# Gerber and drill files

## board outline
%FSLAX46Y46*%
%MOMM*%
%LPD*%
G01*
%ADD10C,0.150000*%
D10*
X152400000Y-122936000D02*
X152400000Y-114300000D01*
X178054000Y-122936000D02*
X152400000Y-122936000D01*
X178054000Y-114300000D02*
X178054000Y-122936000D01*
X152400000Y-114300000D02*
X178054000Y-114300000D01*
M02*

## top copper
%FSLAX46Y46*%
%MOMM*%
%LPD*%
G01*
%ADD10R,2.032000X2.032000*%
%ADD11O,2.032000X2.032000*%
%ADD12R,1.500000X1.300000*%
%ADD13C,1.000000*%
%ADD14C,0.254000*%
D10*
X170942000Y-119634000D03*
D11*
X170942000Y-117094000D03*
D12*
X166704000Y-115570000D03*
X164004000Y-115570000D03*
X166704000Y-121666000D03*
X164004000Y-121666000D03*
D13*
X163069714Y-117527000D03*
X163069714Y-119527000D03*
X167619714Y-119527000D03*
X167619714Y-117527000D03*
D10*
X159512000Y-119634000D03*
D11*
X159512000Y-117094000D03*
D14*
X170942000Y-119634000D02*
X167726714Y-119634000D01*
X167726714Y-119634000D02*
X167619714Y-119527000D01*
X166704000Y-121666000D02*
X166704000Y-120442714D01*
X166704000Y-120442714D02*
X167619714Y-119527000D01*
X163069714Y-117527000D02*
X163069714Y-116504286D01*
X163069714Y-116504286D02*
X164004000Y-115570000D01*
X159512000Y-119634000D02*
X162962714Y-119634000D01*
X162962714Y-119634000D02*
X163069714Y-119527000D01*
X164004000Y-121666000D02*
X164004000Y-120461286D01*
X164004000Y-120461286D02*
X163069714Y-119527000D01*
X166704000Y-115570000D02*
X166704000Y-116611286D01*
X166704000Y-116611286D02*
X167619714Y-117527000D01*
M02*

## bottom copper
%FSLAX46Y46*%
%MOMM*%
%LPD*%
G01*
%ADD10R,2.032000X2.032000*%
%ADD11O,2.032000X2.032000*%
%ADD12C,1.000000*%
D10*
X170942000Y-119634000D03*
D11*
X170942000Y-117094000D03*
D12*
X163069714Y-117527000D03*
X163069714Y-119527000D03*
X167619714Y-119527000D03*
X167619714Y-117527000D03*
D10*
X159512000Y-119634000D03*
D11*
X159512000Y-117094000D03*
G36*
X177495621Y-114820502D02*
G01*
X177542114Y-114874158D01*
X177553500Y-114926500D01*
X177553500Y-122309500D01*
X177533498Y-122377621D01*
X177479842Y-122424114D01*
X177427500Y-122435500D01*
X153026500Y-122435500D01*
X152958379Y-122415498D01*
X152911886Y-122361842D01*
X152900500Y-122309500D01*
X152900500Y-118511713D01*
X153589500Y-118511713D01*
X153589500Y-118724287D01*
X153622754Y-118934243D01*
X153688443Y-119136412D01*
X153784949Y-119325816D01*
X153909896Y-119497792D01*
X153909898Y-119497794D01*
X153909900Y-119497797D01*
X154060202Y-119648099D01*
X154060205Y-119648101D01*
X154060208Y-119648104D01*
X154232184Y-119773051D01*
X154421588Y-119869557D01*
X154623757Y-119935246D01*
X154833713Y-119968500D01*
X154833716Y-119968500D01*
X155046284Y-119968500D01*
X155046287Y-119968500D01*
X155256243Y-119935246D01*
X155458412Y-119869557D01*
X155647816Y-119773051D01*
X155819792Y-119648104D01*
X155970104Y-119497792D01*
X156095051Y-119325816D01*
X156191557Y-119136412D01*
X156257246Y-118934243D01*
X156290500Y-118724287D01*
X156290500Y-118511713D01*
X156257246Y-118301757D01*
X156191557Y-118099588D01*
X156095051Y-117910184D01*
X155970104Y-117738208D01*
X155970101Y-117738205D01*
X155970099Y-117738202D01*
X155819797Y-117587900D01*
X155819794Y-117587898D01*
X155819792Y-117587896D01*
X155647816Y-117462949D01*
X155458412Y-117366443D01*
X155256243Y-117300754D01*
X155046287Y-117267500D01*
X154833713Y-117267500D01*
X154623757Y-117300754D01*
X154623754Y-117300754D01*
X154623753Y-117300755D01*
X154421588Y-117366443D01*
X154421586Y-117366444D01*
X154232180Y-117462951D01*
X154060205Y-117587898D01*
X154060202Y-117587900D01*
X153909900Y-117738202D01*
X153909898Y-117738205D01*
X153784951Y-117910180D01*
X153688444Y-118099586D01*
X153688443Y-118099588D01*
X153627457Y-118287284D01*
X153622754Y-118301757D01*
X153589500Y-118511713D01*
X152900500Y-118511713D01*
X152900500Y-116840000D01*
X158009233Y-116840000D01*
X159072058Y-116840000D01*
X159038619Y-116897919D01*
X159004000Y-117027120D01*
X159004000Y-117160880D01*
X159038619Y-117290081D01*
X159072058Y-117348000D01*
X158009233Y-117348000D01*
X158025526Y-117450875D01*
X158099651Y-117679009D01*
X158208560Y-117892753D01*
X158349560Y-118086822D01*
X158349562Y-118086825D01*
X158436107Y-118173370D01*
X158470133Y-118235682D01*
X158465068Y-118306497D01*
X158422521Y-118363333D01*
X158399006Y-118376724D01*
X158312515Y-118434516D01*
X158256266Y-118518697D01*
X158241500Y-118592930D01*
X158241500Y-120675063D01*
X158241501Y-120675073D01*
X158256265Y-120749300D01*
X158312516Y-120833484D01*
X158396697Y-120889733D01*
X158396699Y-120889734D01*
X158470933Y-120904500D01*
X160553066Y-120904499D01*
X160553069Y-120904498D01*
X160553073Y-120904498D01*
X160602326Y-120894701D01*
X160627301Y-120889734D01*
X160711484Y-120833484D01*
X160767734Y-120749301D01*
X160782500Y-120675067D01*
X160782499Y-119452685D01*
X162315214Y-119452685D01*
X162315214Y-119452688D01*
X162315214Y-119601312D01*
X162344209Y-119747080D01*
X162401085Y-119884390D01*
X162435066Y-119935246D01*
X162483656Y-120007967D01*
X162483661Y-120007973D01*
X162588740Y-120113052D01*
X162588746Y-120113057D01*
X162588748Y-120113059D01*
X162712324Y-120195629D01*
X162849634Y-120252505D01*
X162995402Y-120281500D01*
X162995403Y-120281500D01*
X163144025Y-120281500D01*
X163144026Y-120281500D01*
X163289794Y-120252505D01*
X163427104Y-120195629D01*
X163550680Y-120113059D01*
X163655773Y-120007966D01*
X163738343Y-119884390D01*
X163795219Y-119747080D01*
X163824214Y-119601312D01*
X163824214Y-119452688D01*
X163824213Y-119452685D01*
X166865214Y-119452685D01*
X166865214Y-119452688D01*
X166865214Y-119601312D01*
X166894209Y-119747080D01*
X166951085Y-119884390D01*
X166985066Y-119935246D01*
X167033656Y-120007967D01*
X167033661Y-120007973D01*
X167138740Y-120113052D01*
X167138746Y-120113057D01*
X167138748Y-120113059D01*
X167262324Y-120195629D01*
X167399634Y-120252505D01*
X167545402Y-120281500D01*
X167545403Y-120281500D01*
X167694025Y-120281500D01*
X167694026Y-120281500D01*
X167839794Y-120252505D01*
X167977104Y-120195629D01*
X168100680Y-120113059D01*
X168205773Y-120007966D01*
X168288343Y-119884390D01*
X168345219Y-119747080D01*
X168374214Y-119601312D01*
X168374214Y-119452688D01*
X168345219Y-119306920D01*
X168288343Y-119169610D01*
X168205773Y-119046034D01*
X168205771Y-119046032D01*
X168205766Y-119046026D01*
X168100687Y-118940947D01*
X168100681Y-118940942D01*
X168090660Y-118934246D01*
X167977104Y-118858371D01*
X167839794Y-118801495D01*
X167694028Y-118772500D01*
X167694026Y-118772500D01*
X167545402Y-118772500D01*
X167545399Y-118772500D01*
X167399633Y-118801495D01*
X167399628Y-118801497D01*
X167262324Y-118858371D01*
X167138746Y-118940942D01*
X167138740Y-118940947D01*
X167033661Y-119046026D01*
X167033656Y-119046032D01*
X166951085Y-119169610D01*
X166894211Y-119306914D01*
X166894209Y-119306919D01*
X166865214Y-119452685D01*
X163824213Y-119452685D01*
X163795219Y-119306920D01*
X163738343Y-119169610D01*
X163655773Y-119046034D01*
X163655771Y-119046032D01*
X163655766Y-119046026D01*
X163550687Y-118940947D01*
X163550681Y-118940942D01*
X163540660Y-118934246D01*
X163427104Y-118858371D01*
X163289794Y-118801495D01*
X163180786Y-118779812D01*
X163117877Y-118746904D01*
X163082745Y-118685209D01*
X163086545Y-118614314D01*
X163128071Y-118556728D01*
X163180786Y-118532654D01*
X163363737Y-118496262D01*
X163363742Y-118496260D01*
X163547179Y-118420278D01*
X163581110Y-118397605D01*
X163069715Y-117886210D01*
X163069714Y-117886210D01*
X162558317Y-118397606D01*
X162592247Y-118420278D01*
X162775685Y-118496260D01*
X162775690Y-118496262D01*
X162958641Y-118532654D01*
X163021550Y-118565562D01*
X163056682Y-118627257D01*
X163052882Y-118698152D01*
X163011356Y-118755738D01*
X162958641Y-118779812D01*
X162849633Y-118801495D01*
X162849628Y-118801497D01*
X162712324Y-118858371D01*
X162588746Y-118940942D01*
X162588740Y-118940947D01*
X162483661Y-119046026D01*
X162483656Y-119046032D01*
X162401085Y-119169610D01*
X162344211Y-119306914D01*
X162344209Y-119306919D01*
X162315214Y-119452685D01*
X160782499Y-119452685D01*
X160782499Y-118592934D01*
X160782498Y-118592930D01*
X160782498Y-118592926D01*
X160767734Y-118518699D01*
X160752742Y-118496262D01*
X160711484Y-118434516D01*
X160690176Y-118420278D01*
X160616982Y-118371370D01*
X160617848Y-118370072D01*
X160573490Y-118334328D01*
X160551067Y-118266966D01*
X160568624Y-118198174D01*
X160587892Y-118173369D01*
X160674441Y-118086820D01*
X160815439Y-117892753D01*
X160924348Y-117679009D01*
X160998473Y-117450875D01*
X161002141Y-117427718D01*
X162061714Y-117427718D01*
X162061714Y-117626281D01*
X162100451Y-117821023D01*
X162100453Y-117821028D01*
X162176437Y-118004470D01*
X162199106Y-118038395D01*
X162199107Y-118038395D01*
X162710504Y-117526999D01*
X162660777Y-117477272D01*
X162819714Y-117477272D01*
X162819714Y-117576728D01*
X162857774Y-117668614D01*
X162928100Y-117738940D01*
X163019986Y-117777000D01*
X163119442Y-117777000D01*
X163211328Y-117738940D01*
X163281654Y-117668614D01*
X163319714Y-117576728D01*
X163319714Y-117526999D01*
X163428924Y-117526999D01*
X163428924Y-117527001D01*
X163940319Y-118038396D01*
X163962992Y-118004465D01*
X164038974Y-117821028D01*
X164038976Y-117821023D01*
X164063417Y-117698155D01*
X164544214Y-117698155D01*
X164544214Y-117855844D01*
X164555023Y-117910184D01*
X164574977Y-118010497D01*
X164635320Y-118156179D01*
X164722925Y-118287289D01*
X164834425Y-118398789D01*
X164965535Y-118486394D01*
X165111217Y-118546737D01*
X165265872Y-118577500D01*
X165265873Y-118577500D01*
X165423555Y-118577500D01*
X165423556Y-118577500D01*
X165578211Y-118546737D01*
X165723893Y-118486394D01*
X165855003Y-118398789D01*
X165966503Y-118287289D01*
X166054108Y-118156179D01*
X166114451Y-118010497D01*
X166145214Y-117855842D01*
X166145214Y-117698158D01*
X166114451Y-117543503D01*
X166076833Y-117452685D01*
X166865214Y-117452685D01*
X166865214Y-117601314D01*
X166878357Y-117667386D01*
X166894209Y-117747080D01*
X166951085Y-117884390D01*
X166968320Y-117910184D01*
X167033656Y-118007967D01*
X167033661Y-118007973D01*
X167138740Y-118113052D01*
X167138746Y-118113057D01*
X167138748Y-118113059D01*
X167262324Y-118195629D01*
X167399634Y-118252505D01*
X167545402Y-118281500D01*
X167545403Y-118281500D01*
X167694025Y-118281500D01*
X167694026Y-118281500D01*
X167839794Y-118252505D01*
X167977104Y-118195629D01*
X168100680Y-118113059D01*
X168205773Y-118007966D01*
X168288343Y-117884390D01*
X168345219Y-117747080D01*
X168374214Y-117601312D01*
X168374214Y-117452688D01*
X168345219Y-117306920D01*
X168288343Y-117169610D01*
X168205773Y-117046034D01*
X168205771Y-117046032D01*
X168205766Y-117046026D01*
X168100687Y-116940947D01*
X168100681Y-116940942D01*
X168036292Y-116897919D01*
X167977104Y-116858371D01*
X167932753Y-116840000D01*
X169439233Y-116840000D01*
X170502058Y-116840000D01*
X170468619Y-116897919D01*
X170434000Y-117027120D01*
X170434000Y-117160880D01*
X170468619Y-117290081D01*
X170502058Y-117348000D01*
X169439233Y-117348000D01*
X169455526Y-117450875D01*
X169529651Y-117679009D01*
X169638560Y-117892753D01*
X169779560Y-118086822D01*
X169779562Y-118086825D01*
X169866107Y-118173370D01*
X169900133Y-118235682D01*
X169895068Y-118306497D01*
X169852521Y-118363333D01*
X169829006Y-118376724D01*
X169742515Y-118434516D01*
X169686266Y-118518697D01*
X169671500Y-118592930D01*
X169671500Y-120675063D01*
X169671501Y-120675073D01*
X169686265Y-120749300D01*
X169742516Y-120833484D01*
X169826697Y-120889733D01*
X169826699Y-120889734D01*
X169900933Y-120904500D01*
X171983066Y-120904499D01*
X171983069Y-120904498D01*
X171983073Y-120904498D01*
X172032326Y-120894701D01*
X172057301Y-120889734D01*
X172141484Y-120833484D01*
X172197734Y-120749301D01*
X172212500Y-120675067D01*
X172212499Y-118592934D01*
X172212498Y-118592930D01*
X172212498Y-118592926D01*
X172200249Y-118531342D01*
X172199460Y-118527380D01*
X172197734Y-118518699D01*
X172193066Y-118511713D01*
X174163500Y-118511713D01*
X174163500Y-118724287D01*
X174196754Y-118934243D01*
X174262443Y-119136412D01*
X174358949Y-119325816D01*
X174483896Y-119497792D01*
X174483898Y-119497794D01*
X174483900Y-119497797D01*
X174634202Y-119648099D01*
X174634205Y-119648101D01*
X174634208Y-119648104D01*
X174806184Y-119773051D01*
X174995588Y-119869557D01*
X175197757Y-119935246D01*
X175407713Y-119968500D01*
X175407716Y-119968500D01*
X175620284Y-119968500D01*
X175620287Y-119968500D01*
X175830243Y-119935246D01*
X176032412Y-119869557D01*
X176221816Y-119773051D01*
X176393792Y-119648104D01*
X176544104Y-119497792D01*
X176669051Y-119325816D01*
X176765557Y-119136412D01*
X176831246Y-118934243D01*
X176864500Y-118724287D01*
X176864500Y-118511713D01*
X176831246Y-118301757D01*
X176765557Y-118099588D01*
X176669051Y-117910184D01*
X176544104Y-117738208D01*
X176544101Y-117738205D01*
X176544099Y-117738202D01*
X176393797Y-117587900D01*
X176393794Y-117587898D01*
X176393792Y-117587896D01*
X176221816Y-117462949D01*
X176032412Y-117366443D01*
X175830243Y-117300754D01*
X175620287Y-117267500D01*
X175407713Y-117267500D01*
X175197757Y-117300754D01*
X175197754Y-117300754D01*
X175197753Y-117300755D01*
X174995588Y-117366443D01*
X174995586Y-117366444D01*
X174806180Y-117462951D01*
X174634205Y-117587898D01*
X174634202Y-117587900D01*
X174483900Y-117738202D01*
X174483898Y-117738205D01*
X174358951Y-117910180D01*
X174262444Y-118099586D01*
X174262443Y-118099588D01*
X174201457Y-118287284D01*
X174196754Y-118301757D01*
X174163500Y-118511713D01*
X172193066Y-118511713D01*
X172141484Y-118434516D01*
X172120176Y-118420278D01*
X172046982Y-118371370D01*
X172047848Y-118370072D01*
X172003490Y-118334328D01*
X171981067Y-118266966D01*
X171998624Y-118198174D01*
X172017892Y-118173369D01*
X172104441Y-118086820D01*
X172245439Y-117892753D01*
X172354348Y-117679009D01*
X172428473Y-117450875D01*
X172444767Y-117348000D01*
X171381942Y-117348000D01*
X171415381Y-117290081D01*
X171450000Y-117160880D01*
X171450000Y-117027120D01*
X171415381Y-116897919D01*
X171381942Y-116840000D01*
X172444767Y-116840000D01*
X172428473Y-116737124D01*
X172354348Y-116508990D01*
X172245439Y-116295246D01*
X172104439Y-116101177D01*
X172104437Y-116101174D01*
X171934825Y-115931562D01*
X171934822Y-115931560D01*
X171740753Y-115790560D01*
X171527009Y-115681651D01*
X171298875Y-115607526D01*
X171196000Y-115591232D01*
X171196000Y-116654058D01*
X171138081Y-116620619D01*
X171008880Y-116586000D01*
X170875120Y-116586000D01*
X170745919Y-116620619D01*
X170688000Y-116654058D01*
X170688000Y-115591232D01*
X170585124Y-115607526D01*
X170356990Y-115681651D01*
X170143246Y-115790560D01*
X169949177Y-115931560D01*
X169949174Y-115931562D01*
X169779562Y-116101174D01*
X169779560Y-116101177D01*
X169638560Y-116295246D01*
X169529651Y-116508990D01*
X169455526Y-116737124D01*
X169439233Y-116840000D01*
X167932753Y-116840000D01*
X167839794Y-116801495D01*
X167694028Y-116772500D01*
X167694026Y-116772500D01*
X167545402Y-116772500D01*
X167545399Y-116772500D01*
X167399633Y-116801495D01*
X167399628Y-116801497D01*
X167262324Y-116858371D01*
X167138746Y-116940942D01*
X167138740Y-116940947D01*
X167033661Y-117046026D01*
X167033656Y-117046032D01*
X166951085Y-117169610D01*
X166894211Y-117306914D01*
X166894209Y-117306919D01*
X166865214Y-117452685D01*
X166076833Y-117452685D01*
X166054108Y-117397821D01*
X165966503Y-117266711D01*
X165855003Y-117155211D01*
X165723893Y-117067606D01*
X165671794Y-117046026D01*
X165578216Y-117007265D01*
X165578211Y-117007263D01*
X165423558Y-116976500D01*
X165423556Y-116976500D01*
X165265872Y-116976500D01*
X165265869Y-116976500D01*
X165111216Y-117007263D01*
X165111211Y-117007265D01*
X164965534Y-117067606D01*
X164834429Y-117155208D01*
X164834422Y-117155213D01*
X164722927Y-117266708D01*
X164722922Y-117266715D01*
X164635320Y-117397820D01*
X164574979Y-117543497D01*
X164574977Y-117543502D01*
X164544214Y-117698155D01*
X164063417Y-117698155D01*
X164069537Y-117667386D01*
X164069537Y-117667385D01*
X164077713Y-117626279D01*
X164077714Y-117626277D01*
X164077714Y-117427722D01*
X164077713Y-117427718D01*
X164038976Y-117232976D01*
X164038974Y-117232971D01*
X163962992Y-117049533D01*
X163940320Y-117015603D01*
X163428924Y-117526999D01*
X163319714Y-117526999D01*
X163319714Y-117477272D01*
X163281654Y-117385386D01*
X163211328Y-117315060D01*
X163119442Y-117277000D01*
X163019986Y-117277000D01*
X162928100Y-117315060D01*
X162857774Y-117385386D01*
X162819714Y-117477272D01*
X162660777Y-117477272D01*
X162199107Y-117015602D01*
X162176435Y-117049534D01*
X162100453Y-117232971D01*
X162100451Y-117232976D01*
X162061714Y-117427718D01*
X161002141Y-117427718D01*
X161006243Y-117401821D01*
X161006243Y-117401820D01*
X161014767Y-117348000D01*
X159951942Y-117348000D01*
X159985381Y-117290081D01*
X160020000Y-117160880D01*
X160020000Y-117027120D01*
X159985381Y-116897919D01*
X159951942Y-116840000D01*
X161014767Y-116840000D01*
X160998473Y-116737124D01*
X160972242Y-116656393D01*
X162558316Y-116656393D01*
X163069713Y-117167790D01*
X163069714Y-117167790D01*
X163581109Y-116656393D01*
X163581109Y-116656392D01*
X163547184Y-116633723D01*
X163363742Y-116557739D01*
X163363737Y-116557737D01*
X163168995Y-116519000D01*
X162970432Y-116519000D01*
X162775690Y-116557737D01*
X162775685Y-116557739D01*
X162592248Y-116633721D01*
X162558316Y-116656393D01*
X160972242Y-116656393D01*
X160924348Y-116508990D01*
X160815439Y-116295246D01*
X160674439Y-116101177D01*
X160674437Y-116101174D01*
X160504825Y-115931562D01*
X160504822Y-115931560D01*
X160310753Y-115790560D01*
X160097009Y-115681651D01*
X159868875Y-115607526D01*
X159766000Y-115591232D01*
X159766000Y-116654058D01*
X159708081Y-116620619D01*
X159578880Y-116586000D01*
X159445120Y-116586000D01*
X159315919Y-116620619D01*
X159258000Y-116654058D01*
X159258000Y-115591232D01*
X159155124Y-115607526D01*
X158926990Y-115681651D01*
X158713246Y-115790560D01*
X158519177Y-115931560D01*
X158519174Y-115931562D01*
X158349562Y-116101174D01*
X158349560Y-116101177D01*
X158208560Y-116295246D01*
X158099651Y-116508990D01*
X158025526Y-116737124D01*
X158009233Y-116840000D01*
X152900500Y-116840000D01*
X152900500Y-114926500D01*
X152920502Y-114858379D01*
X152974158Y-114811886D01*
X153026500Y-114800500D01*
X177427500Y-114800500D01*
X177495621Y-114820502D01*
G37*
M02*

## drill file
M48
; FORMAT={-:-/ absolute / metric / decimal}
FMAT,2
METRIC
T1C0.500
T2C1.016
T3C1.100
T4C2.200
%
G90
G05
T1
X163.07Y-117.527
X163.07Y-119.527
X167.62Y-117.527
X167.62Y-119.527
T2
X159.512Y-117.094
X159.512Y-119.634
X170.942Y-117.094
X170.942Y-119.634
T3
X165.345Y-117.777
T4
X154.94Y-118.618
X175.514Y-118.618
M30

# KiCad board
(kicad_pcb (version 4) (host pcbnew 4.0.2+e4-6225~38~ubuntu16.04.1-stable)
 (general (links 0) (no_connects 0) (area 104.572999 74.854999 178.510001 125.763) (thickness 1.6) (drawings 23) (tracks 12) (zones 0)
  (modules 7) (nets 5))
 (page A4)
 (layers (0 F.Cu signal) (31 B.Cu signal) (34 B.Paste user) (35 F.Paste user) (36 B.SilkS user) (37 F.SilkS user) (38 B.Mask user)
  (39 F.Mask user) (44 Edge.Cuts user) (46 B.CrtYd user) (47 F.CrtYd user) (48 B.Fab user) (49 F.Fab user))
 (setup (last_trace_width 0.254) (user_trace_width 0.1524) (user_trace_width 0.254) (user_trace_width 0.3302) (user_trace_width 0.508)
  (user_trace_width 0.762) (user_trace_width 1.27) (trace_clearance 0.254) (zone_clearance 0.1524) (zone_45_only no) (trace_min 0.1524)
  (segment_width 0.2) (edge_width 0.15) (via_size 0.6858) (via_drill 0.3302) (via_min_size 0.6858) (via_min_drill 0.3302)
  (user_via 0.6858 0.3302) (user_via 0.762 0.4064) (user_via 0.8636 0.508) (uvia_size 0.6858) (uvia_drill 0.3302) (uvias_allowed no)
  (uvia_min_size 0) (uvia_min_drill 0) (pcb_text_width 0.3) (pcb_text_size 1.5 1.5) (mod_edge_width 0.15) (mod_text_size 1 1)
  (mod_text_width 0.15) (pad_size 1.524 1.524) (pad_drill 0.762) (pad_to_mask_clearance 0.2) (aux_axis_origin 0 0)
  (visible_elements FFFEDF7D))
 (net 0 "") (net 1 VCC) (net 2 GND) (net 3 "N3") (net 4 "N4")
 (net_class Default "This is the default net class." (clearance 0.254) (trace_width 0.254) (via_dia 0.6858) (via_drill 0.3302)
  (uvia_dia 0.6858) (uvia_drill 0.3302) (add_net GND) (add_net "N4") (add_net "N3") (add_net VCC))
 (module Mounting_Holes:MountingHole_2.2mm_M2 (layer F.Cu) (at 175.514 118.618)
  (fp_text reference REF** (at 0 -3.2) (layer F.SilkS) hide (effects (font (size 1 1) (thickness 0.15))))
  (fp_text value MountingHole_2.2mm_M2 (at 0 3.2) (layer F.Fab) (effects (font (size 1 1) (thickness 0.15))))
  (pad 1 np_thru_hole circle (at 0 0) (size 2.2 2.2) (drill 2.2) (layers *.Cu *.Mask F.SilkS)))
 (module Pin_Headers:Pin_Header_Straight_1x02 (layer F.Cu) (at 170.942 119.634 180)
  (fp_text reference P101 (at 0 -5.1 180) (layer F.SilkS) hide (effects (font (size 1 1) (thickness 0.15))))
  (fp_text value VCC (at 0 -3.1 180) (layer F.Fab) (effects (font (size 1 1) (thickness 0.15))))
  (pad 1 thru_hole rect (at 0 0 180) (size 2.032 2.032) (drill 1.016) (layers *.Cu *.Mask F.SilkS) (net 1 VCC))
  (pad 2 thru_hole oval (at 0 2.54 180) (size 2.032 2.032) (drill 1.016) (layers *.Cu *.Mask F.SilkS) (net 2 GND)))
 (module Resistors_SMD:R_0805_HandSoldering (layer F.Cu) (at 165.354 115.57 180)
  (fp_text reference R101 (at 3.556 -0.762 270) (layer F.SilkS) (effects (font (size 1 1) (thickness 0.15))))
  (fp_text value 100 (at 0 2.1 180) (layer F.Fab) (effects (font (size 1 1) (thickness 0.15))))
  (pad 1 smd rect (at -1.35 0 180) (size 1.5 1.3) (layers F.Cu F.Paste F.Mask) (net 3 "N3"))
  (pad 2 smd rect (at 1.35 0 180) (size 1.5 1.3) (layers F.Cu F.Paste F.Mask) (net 2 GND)))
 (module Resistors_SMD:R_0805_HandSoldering (layer F.Cu) (at 165.354 121.666 180)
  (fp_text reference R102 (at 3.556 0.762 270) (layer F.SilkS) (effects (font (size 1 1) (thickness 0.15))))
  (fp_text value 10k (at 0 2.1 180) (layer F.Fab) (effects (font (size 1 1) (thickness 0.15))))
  (pad 1 smd rect (at -1.35 0 180) (size 1.5 1.3) (layers F.Cu F.Paste F.Mask) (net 1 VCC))
  (pad 2 smd rect (at 1.35 0 180) (size 1.5 1.3) (layers F.Cu F.Paste F.Mask) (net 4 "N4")))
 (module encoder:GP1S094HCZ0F (layer F.Cu) (at 165.344714 118.527)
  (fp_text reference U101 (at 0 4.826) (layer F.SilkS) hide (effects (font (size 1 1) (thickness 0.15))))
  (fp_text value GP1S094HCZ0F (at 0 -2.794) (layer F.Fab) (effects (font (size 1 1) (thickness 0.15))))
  (pad 3 thru_hole circle (at -2.275 -1) (size 1 1) (drill 0.5) (layers *.Cu *.Mask F.SilkS) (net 2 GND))
  (pad 2 thru_hole circle (at -2.275 1) (size 1 1) (drill 0.5) (layers *.Cu *.Mask F.SilkS) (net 4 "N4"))
  (pad 1 thru_hole circle (at 2.275 1) (size 1 1) (drill 0.5) (layers *.Cu *.Mask F.SilkS) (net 1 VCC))
  (pad 4 thru_hole circle (at 2.275 -1) (size 1 1) (drill 0.5) (layers *.Cu *.Mask F.SilkS) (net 3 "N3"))
  (pad "" np_thru_hole circle (at 0 -0.75) (size 1.1 1.1) (drill 1.1) (layers *.Cu *.Mask F.SilkS)))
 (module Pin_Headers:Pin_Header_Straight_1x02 (layer F.Cu) (at 159.512 119.634 180)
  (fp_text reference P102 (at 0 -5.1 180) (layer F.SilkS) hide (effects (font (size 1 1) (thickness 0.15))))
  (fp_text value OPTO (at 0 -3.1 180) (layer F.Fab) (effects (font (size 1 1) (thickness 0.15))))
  (pad 1 thru_hole rect (at 0 0 180) (size 2.032 2.032) (drill 1.016) (layers *.Cu *.Mask F.SilkS) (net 4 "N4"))
  (pad 2 thru_hole oval (at 0 2.54 180) (size 2.032 2.032) (drill 1.016) (layers *.Cu *.Mask F.SilkS) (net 2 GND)))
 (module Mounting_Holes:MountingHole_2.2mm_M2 (layer F.Cu) (at 154.94 118.618)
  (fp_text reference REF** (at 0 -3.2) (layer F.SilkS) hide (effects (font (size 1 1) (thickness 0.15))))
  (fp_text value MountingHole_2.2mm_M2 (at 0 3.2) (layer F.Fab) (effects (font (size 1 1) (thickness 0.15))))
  (pad 1 np_thru_hole circle (at 0 0) (size 2.2 2.2) (drill 2.2) (layers *.Cu *.Mask F.SilkS)))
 (gr_line (start 152.4 122.936) (end 152.4 114.3) (layer Edge.Cuts) (width 0.15))
 (gr_line (start 178.054 122.936) (end 152.4 122.936) (layer Edge.Cuts) (width 0.15))
 (gr_line (start 178.054 114.3) (end 178.054 122.936) (layer Edge.Cuts) (width 0.15))
 (gr_line (start 152.4 114.3) (end 178.054 114.3) (layer Edge.Cuts) (width 0.15))
 (segment (start 170.942 119.634) (end 167.726714 119.634) (width 0.254) (layer F.Cu) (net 1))
 (segment (start 167.726714 119.634) (end 167.619714 119.527) (width 0.254) (layer F.Cu) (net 1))
 (segment (start 166.704 121.666) (end 166.704 120.442714) (width 0.254) (layer F.Cu) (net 1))
 (segment (start 166.704 120.442714) (end 167.619714 119.527) (width 0.254) (layer F.Cu) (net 1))
 (segment (start 163.069714 117.527) (end 163.069714 116.504286) (width 0.254) (layer F.Cu) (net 2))
 (segment (start 163.069714 116.504286) (end 164.004 115.57) (width 0.254) (layer F.Cu) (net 2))
 (segment (start 159.512 119.634) (end 162.962714 119.634) (width 0.254) (layer F.Cu) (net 4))
 (segment (start 162.962714 119.634) (end 163.069714 119.527) (width 0.254) (layer F.Cu) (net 4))
 (segment (start 164.004 121.666) (end 164.004 120.461286) (width 0.254) (layer F.Cu) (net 4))
 (segment (start 164.004 120.461286) (end 163.069714 119.527) (width 0.254) (layer F.Cu) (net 4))
 (segment (start 166.704 115.57) (end 166.704 116.611286) (width 0.254) (layer F.Cu) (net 3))
 (segment (start 166.704 116.611286) (end 167.619714 117.527) (width 0.254) (layer F.Cu) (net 3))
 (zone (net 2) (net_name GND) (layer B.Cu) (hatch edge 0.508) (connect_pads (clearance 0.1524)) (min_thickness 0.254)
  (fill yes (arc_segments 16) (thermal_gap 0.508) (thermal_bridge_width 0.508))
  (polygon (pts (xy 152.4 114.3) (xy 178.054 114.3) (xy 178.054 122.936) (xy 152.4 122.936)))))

